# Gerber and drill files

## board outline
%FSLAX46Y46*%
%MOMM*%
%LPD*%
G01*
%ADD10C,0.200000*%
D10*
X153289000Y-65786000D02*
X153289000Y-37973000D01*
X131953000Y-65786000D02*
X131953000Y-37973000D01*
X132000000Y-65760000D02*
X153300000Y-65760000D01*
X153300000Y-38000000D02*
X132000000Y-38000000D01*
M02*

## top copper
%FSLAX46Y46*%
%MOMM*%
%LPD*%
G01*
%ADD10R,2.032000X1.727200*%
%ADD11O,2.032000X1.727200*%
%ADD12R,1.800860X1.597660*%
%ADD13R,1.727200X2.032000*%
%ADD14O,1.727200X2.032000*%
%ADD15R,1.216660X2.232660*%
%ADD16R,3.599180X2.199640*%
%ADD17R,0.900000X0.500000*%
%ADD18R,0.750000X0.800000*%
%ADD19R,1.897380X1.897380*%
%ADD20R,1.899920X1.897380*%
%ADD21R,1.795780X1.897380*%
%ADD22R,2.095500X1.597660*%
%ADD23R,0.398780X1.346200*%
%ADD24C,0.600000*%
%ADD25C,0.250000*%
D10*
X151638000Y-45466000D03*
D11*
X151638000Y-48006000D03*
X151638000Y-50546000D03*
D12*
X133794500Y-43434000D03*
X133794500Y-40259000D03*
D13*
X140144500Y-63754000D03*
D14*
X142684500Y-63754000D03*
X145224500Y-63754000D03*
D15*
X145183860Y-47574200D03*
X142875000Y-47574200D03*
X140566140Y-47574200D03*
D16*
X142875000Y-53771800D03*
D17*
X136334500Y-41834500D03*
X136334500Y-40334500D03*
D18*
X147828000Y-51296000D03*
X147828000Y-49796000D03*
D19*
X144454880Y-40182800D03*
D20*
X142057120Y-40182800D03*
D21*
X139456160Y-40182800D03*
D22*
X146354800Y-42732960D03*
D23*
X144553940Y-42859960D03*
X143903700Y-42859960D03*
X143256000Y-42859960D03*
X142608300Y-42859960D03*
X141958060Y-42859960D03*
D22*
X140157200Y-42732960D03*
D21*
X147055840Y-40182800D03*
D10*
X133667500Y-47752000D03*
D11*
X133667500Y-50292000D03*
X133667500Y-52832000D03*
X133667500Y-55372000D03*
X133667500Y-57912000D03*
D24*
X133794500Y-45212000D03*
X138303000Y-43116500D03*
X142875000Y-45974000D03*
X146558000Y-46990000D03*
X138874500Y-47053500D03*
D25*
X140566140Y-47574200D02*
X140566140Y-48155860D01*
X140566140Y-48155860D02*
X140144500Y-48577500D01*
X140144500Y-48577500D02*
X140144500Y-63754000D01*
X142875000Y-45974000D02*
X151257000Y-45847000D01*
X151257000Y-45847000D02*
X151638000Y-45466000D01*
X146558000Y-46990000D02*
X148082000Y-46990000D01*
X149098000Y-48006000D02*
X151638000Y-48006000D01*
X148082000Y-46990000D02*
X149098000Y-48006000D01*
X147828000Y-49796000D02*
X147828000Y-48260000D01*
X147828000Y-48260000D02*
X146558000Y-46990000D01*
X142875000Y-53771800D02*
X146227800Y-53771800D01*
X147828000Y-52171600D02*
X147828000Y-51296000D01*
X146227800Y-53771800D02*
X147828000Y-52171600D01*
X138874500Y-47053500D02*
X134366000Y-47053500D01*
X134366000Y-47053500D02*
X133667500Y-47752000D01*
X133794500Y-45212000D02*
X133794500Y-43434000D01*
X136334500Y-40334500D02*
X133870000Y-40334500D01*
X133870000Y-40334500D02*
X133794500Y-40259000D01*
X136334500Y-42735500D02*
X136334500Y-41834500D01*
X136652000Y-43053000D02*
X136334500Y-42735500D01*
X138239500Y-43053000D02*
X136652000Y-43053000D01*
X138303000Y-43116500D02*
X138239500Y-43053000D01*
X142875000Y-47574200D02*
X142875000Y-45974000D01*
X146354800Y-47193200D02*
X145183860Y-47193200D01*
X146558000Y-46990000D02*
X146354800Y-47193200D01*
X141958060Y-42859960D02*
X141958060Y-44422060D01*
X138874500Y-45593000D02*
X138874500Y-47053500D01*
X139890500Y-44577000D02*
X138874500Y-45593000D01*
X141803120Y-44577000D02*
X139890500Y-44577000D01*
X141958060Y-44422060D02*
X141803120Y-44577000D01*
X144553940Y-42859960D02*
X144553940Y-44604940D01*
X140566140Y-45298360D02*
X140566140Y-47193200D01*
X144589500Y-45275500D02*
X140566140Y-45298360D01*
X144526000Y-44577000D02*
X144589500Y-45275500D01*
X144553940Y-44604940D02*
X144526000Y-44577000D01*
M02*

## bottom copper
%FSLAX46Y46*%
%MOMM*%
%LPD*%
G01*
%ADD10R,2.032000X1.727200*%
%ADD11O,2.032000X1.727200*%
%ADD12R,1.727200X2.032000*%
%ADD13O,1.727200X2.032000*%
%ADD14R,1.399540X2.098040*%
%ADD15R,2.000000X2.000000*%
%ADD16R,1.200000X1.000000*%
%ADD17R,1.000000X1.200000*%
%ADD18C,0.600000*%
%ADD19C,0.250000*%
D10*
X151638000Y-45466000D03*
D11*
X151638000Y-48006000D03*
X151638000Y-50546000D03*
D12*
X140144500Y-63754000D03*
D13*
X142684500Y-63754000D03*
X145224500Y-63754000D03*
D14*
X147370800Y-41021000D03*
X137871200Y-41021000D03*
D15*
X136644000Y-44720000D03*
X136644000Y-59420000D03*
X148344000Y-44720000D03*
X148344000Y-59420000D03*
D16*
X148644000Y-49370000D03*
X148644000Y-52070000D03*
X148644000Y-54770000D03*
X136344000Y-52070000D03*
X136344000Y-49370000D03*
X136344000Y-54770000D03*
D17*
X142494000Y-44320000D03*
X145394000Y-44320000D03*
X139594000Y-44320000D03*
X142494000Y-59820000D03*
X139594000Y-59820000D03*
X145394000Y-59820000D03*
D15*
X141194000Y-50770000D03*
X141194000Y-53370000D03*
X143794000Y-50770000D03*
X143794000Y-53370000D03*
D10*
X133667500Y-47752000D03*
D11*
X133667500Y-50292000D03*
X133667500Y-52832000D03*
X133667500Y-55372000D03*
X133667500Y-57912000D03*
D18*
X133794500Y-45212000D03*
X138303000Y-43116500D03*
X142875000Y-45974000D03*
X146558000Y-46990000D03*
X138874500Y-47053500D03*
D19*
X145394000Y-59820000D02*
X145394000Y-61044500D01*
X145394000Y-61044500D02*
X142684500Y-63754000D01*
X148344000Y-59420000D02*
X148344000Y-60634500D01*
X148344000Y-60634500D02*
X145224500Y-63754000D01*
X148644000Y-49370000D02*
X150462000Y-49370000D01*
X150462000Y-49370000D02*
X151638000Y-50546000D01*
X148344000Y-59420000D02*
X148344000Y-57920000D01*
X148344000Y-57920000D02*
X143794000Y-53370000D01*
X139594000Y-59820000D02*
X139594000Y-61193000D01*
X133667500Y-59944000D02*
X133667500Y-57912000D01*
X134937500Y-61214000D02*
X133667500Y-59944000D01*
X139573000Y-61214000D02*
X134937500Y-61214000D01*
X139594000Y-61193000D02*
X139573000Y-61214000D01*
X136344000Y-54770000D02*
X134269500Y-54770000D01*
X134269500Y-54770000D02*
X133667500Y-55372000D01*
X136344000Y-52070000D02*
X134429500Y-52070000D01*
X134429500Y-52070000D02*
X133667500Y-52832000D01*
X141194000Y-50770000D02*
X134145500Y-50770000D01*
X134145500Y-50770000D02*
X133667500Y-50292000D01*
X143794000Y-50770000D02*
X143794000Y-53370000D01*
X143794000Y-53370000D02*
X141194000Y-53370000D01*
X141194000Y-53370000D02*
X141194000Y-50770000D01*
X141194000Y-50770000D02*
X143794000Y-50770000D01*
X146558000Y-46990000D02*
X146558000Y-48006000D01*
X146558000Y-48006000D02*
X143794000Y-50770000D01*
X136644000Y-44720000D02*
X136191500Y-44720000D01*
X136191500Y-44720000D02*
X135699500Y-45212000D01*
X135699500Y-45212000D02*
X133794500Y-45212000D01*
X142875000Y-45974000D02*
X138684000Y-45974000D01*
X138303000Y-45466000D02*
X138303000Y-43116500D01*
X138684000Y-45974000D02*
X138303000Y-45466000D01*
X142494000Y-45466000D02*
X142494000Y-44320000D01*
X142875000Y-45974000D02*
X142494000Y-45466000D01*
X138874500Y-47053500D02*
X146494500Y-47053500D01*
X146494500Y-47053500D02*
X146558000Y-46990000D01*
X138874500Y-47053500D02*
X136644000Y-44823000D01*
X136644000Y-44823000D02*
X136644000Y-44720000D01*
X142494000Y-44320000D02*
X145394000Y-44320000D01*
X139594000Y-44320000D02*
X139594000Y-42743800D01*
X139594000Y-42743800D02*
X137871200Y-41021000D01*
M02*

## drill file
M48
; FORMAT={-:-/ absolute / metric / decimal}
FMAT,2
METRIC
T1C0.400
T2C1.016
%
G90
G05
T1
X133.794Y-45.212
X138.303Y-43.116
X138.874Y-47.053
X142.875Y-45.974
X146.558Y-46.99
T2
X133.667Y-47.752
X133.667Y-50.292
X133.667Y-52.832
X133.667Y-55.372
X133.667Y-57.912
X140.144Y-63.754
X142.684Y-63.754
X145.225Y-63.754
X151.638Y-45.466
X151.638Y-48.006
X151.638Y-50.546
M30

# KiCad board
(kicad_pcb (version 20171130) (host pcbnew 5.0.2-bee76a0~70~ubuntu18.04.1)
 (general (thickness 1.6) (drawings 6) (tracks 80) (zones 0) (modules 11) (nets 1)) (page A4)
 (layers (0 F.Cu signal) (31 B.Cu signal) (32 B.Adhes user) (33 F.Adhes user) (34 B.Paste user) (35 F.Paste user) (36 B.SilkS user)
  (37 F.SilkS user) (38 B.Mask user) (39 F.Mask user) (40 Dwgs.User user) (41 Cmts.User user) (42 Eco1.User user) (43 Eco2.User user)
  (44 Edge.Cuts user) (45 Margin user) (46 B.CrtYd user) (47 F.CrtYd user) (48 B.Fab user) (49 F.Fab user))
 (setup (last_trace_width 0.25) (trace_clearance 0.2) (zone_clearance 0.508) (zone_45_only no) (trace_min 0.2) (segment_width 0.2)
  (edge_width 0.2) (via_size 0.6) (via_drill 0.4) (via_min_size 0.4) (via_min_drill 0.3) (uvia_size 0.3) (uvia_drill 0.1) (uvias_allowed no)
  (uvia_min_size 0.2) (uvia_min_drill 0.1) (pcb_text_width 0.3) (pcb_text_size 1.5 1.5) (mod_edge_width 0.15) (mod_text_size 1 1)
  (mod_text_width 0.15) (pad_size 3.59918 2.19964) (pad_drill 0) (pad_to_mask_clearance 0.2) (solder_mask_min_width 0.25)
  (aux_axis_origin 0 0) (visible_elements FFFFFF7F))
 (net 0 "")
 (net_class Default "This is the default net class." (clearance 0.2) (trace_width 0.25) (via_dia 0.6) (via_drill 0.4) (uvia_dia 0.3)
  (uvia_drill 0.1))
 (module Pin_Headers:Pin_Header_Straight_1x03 (layer F.Cu) (at 151.638 45.466)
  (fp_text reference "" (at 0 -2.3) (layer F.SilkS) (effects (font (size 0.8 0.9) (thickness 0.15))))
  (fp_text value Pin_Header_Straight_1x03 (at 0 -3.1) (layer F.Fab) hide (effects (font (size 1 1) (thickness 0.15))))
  (pad 1 thru_hole rect (at 0 0) (size 2.032 1.7272) (drill 1.016) (layers *.Cu *.Mask F.SilkS))
  (pad 2 thru_hole oval (at 0 2.54) (size 2.032 1.7272) (drill 1.016) (layers *.Cu *.Mask F.SilkS))
  (pad 3 thru_hole oval (at 0 5.08) (size 2.032 1.7272) (drill 1.016) (layers *.Cu *.Mask F.SilkS)))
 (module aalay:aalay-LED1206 (layer F.Cu) (at 133.7945 41.8465 90)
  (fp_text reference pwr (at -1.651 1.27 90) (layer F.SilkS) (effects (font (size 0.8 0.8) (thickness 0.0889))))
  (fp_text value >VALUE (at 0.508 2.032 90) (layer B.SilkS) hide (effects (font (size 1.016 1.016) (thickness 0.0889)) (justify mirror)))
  (pad A smd rect (at -1.5875 0 90) (size 1.59766 1.80086) (layers F.Cu F.Paste F.Mask))
  (pad K smd rect (at 1.5875 0 90) (size 1.59766 1.80086) (layers F.Cu F.Paste F.Mask)))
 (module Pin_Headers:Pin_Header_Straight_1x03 (layer F.Cu) (at 140.1445 63.754 90)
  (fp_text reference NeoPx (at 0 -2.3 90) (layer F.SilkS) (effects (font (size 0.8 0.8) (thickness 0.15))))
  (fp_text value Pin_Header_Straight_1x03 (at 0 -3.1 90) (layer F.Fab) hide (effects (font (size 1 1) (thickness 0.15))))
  (pad 1 thru_hole rect (at 0 0 90) (size 2.032 1.7272) (drill 1.016) (layers *.Cu *.Mask F.SilkS))
  (pad 2 thru_hole oval (at 0 2.54 90) (size 2.032 1.7272) (drill 1.016) (layers *.Cu *.Mask F.SilkS))
  (pad 3 thru_hole oval (at 0 5.08 90) (size 2.032 1.7272) (drill 1.016) (layers *.Cu *.Mask F.SilkS)))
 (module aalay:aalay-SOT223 (layer F.Cu) (at 142.875 50.673 180)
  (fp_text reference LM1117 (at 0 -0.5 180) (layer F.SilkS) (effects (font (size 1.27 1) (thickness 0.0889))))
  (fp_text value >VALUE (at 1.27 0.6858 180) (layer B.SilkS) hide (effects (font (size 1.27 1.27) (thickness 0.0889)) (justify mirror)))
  (pad GND smd rect (at -2.30886 3.0988 180) (size 1.21666 2.23266) (layers F.Cu F.Paste F.Mask))
  (pad OUT smd rect (at 0 3.0988 180) (size 1.21666 2.23266) (layers F.Cu F.Paste F.Mask))
  (pad IN smd rect (at 2.30886 3.0988 180) (size 1.21666 2.23266) (layers F.Cu F.Paste F.Mask))
  (pad OUT smd rect (at 0 -3.0988 180) (size 3.59918 2.19964) (layers F.Cu F.Paste F.Mask)))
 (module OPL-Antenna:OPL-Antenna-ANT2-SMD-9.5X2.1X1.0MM (layer B.Cu) (at 142.621 41.021 180)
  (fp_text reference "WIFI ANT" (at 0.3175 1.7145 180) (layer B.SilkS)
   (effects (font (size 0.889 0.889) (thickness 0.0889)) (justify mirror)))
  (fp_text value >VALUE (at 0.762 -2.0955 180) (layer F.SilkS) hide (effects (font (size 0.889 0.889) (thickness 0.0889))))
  (pad 1 smd rect (at -4.7498 0 180) (size 1.39954 2.09804) (layers B.Cu B.Paste B.Mask))
  (pad 2 smd rect (at 4.7498 0 180) (size 1.39954 2.09804) (layers B.Cu B.Paste B.Mask)))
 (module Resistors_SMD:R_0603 (layer F.Cu) (at 136.3345 41.0845 90)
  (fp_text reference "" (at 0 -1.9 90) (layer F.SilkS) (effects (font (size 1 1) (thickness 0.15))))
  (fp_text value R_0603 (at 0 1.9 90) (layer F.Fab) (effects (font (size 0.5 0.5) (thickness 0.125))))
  (pad 1 smd rect (at -0.75 0 90) (size 0.5 0.9) (layers F.Cu F.Paste F.Mask))
  (pad 2 smd rect (at 0.75 0 90) (size 0.5 0.9) (layers F.Cu F.Paste F.Mask)))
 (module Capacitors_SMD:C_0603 (layer F.Cu) (at 147.828 50.546 90)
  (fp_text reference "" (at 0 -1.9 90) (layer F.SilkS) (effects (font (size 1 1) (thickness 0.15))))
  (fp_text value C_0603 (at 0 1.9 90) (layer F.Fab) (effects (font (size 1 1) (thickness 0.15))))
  (pad 1 smd rect (at -0.75 0 90) (size 0.8 0.75) (layers F.Cu F.Paste F.Mask))
  (pad 2 smd rect (at 0.75 0 90) (size 0.8 0.75) (layers F.Cu F.Paste F.Mask)))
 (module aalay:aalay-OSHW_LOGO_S (layer F.Cu) (at 150.622 39.878)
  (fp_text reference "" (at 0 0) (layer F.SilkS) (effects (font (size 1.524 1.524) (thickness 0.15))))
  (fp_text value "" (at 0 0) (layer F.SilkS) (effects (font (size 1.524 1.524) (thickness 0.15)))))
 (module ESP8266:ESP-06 (layer B.Cu) (at 142.494 52.07 270)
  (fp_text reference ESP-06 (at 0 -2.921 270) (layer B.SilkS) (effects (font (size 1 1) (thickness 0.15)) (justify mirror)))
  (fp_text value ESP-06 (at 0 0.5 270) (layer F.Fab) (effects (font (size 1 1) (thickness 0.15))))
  (pad GND smd rect (at -7.35 5.85 270) (size 2 2) (layers B.Cu B.Paste B.Mask))
  (pad GP5 smd rect (at 7.35 5.85 270) (size 2 2) (layers B.Cu B.Paste B.Mask))
  (pad GP16 smd rect (at -7.35 -5.85 270) (size 2 2) (layers B.Cu B.Paste B.Mask))
  (pad GP15 smd rect (at 7.35 -5.85 270) (size 2 2) (layers B.Cu B.Paste B.Mask))
  (pad GP14 smd rect (at -2.7 -6.15 270) (size 1 1.2) (layers B.Cu B.Paste B.Mask))
  (pad GP12 smd rect (at 0 -6.15 270) (size 1 1.2) (layers B.Cu B.Paste B.Mask))
  (pad GP13 smd rect (at 2.7 -6.15 270) (size 1 1.2) (layers B.Cu B.Paste B.Mask))
  (pad TX smd rect (at 0 6.15 270) (size 1 1.2) (layers B.Cu B.Paste B.Mask))
  (pad RST smd rect (at -2.7 6.15 270) (size 1 1.2) (layers B.Cu B.Paste B.Mask))
  (pad RX smd rect (at 2.7 6.15 270) (size 1 1.2) (layers B.Cu B.Paste B.Mask))
  (pad 3.3 smd rect (at -7.75 0 270) (size 1.2 1) (layers B.Cu B.Paste B.Mask))
  (pad CHPD smd rect (at -7.75 -2.9 270) (size 1.2 1) (layers B.Cu B.Paste B.Mask))
  (pad ANT smd rect (at -7.75 2.9 270) (size 1.2 1) (layers B.Cu B.Paste B.Mask))
  (pad GP2 smd rect (at 7.75 0 270) (size 1.2 1) (layers B.Cu B.Paste B.Mask))
  (pad GP0 smd rect (at 7.75 2.9 270) (size 1.2 1) (layers B.Cu B.Paste B.Mask))
  (pad GP4 smd rect (at 7.75 -2.9 270) (size 1.2 1) (layers B.Cu B.Paste B.Mask))
  (pad GND smd rect (at -1.3 1.3 270) (size 2 2) (layers B.Cu B.Paste B.Mask))
  (pad GND smd rect (at 1.3 1.3 270) (size 2 2) (layers B.Cu B.Paste B.Mask))
  (pad GND smd rect (at -1.3 -1.3 270) (size 2 2) (layers B.Cu B.Paste B.Mask))
  (pad GND smd rect (at 1.3 -1.3 270) (size 2 2) (layers B.Cu B.Paste B.Mask)))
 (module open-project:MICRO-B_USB (layer F.Cu) (at 143.256 38.735 180)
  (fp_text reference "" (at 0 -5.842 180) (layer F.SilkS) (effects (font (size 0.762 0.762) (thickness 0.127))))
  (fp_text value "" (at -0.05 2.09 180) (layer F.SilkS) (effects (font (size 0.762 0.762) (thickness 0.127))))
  (pad "" smd rect (at -1.19888 -1.4478 180) (size 1.89738 1.89738) (layers F.Cu F.Paste F.Mask))
  (pad "" smd rect (at 1.19888 -1.4478 180) (size 1.89992 1.89738) (layers F.Cu F.Paste F.Mask))
  (pad "" smd rect (at 3.79984 -1.4478 180) (size 1.79578 1.89738) (layers F.Cu F.Paste F.Mask))
  (pad "" smd rect (at -3.0988 -3.99796 180) (size 2.0955 1.59766) (layers F.Cu F.Paste F.Mask))
  (pad 1 smd rect (at -1.29794 -4.12496 180) (size 0.39878 1.3462) (layers F.Cu F.Paste F.Mask) (clearance 0.2032))
  (pad 2 smd rect (at -0.6477 -4.12496 180) (size 0.39878 1.3462) (layers F.Cu F.Paste F.Mask) (clearance 0.2032))
  (pad 3 smd rect (at 0 -4.12496 180) (size 0.39878 1.3462) (layers F.Cu F.Paste F.Mask) (clearance 0.2032))
  (pad 4 smd rect (at 0.6477 -4.12496 180) (size 0.39878 1.3462) (layers F.Cu F.Paste F.Mask) (clearance 0.2032))
  (pad 5 smd rect (at 1.29794 -4.12496 180) (size 0.39878 1.3462) (layers F.Cu F.Paste F.Mask) (clearance 0.2032))
  (pad "" smd rect (at 3.0988 -3.99796 180) (size 2.0955 1.59766) (layers F.Cu F.Paste F.Mask))
  (pad "" smd rect (at -3.79984 -1.4478 180) (size 1.79578 1.89738) (layers F.Cu F.Paste F.Mask)))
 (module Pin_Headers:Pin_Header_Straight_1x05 (layer F.Cu) (at 133.6675 47.752)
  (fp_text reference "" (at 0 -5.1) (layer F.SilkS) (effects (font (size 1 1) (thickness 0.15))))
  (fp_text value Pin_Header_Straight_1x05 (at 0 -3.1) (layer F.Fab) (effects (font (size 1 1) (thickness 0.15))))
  (pad 1 thru_hole rect (at 0 0) (size 2.032 1.7272) (drill 1.016) (layers *.Cu *.Mask F.SilkS))
  (pad 2 thru_hole oval (at 0 2.54) (size 2.032 1.7272) (drill 1.016) (layers *.Cu *.Mask F.SilkS))
  (pad 3 thru_hole oval (at 0 5.08) (size 2.032 1.7272) (drill 1.016) (layers *.Cu *.Mask F.SilkS))
  (pad 4 thru_hole oval (at 0 7.62) (size 2.032 1.7272) (drill 1.016) (layers *.Cu *.Mask F.SilkS))
  (pad 5 thru_hole oval (at 0 10.16) (size 2.032 1.7272) (drill 1.016) (layers *.Cu *.Mask F.SilkS)))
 (gr_line (start 153.289 65.786) (end 153.289 37.973) (angle 90) (layer Edge.Cuts) (width 0.2))
 (gr_line (start 131.953 65.786) (end 131.953 37.973) (angle 90) (layer Edge.Cuts) (width 0.2))
 (gr_line (start 132 65.76) (end 153.3 65.76) (angle 90) (layer Edge.Cuts) (width 0.2))
 (gr_line (start 153.3 38) (end 132 38) (angle 90) (layer Edge.Cuts) (width 0.2))
 (segment (start 140.56614 47.5742) (end 140.56614 48.15586) (width 0.25) (layer F.Cu) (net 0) (status C00000))
 (segment (start 140.56614 48.15586) (end 140.1445 48.5775) (width 0.25) (layer F.Cu) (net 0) (status C00000))
 (segment (start 140.1445 48.5775) (end 140.1445 63.754) (width 0.25) (layer F.Cu) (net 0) (status C00000))
 (segment (start 145.394 59.82) (end 145.394 61.0445) (width 0.25) (layer B.Cu) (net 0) (status 400000))
 (segment (start 145.394 61.0445) (end 142.6845 63.754) (width 0.25) (layer B.Cu) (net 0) (status 800000))
 (segment (start 148.344 59.42) (end 148.344 60.6345) (width 0.25) (layer B.Cu) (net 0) (status 400000))
 (segment (start 148.344 60.6345) (end 145.2245 63.754) (width 0.25) (layer B.Cu) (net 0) (status 800000))
 (segment (start 148.644 49.37) (end 150.462 49.37) (width 0.25) (layer B.Cu) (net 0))
 (segment (start 150.462 49.37) (end 151.638 50.546) (width 0.25) (layer B.Cu) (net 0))
 (segment (start 142.875 45.974) (end 151.257 45.847) (width 0.25) (layer F.Cu) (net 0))
 (segment (start 151.257 45.847) (end 151.638 45.466) (width 0.25) (layer F.Cu) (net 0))
 (segment (start 146.558 46.99) (end 148.082 46.99) (width 0.25) (layer F.Cu) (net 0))
 (segment (start 149.098 48.006) (end 151.638 48.006) (width 0.25) (layer F.Cu) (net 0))
 (segment (start 148.082 46.99) (end 149.098 48.006) (width 0.25) (layer F.Cu) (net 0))
 (segment (start 147.828 49.796) (end 147.828 48.26) (width 0.25) (layer F.Cu) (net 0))
 (segment (start 147.828 48.26) (end 146.558 46.99) (width 0.25) (layer F.Cu) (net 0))
 (segment (start 142.875 53.7718) (end 146.2278 53.7718) (width 0.25) (layer F.Cu) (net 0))
 (segment (start 147.828 52.1716) (end 147.828 51.296) (width 0.25) (layer F.Cu) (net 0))
 (segment (start 146.2278 53.7718) (end 147.828 52.1716) (width 0.25) (layer F.Cu) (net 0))
 (segment (start 148.344 59.42) (end 148.344 57.92) (width 0.25) (layer B.Cu) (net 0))
 (segment (start 148.344 57.92) (end 143.794 53.37) (width 0.25) (layer B.Cu) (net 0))
 (segment (start 139.594 59.82) (end 139.594 61.193) (width 0.25) (layer B.Cu) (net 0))
 (segment (start 133.6675 59.944) (end 133.6675 57.912) (width 0.25) (layer B.Cu) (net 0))
 (segment (start 134.9375 61.214) (end 133.6675 59.944) (width 0.25) (layer B.Cu) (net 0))
 (segment (start 139.573 61.214) (end 134.9375 61.214) (width 0.25) (layer B.Cu) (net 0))
 (segment (start 139.594 61.193) (end 139.573 61.214) (width 0.25) (layer B.Cu) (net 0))
 (segment (start 136.344 54.77) (end 134.2695 54.77) (width 0.25) (layer B.Cu) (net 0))
 (segment (start 134.2695 54.77) (end 133.6675 55.372) (width 0.25) (layer B.Cu) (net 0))
 (segment (start 136.344 52.07) (end 134.4295 52.07) (width 0.25) (layer B.Cu) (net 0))
 (segment (start 134.4295 52.07) (end 133.6675 52.832) (width 0.25) (layer B.Cu) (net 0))
 (segment (start 141.194 50.77) (end 134.1455 50.77) (width 0.25) (layer B.Cu) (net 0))
 (segment (start 134.1455 50.77) (end 133.6675 50.292) (width 0.25) (layer B.Cu) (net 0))
 (segment (start 138.8745 47.0535) (end 134.366 47.0535) (width 0.25) (layer F.Cu) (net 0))
 (segment (start 134.366 47.0535) (end 133.6675 47.752) (width 0.25) (layer F.Cu) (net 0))
 (segment (start 143.794 50.77) (end 143.794 53.37) (width 0.25) (layer B.Cu) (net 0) (status 30))
 (segment (start 143.794 53.37) (end 141.194 53.37) (width 0.25) (layer B.Cu) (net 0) (status 30))
 (segment (start 141.194 53.37) (end 141.194 50.77) (width 0.25) (layer B.Cu) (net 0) (status 30))
 (segment (start 141.194 50.77) (end 143.794 50.77) (width 0.25) (layer B.Cu) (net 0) (status 30))
 (segment (start 146.558 46.99) (end 146.558 48.006) (width 0.25) (layer B.Cu) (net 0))
 (segment (start 146.558 48.006) (end 143.794 50.77) (width 0.25) (layer B.Cu) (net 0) (status 20))
 (segment (start 136.644 44.72) (end 136.1915 44.72) (width 0.25) (layer B.Cu) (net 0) (status 30))
 (segment (start 136.1915 44.72) (end 135.6995 45.212) (width 0.25) (layer B.Cu) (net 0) (status 30))
 (segment (start 135.6995 45.212) (end 133.7945 45.212) (width 0.25) (layer B.Cu) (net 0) (status 10))
 (via (at 133.7945 45.212) (size 0.6) (drill 0.4) (layers F.Cu B.Cu) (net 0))
 (segment (start 133.7945 45.212) (end 133.7945 43.434) (width 0.25) (layer F.Cu) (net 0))
 (segment (start 136.3345 40.3345) (end 133.87 40.3345) (width 0.25) (layer F.Cu) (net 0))
 (segment (start 133.87 40.3345) (end 133.7945 40.259) (width 0.25) (layer F.Cu) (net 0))
 (segment (start 142.875 45.974) (end 138.684 45.974) (width 0.25) (layer B.Cu) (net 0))
 (segment (start 136.3345 42.7355) (end 136.3345 41.8345) (width 0.25) (layer F.Cu) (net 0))
 (segment (start 136.652 43.053) (end 136.3345 42.7355) (width 0.25) (layer F.Cu) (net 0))
 (segment (start 138.2395 43.053) (end 136.652 43.053) (width 0.25) (layer F.Cu) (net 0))
 (segment (start 138.303 43.1165) (end 138.2395 43.053) (width 0.25) (layer F.Cu) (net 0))
 (via (at 138.303 43.1165) (size 0.6) (drill 0.4) (layers F.Cu B.Cu) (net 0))
 (segment (start 138.303 45.466) (end 138.303 43.1165) (width 0.25) (layer B.Cu) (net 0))
 (segment (start 138.684 45.974) (end 138.303 45.466) (width 0.25) (layer B.Cu) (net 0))
 (segment (start 142.875 47.5742) (end 142.875 45.974) (width 0.25) (layer F.Cu) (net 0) (status 400010))
 (segment (start 142.494 45.466) (end 142.494 44.32) (width 0.25) (layer B.Cu) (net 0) (status 20))
 (segment (start 142.875 45.974) (end 142.494 45.466) (width 0.25) (layer B.Cu) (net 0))
 (via (at 142.875 45.974) (size 0.6) (drill 0.4) (layers F.Cu B.Cu) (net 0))
 (segment (start 138.8745 47.0535) (end 146.4945 47.0535) (width 0.25) (layer B.Cu) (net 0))
 (segment (start 146.3548 47.1932) (end 145.18386 47.1932) (width 0.25) (layer F.Cu) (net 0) (status 20))
 (segment (start 146.558 46.99) (end 146.3548 47.1932) (width 0.25) (layer F.Cu) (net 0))
 (via (at 146.558 46.99) (size 0.6) (drill 0.4) (layers F.Cu B.Cu) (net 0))
 (segment (start 146.4945 47.0535) (end 146.558 46.99) (width 0.25) (layer B.Cu) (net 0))
 (segment (start 141.95806 42.85996) (end 141.95806 44.42206) (width 0.25) (layer F.Cu) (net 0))
 (segment (start 138.8745 47.0535) (end 136.644 44.823) (width 0.25) (layer B.Cu) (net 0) (status 20))
 (via (at 138.8745 47.0535) (size 0.6) (drill 0.4) (layers F.Cu B.Cu) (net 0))
 (segment (start 138.8745 45.593) (end 138.8745 47.0535) (width 0.25) (layer F.Cu) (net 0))
 (segment (start 139.8905 44.577) (end 138.8745 45.593) (width 0.25) (layer F.Cu) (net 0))
 (segment (start 141.80312 44.577) (end 139.8905 44.577) (width 0.25) (layer F.Cu) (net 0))
 (segment (start 141.95806 44.42206) (end 141.80312 44.577) (width 0.25) (layer F.Cu) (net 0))
 (segment (start 136.644 44.823) (end 136.644 44.72) (width 0.25) (layer B.Cu) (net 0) (status 30))
 (segment (start 144.55394 42.85996) (end 144.55394 44.60494) (width 0.25) (layer F.Cu) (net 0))
 (segment (start 140.56614 45.29836) (end 140.56614 47.1932) (width 0.25) (layer F.Cu) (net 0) (status 20))
 (segment (start 144.5895 45.2755) (end 140.56614 45.29836) (width 0.25) (layer F.Cu) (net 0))
 (segment (start 144.526 44.577) (end 144.5895 45.2755) (width 0.25) (layer F.Cu) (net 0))
 (segment (start 144.55394 44.60494) (end 144.526 44.577) (width 0.25) (layer F.Cu) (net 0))
 (segment (start 142.494 44.32) (end 145.394 44.32) (width 0.25) (layer B.Cu) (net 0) (status 30))
 (segment (start 139.594 44.32) (end 139.594 42.7438) (width 0.25) (layer B.Cu) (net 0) (status 10))
 (segment (start 139.594 42.7438) (end 137.8712 41.021) (width 0.25) (layer B.Cu) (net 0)))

